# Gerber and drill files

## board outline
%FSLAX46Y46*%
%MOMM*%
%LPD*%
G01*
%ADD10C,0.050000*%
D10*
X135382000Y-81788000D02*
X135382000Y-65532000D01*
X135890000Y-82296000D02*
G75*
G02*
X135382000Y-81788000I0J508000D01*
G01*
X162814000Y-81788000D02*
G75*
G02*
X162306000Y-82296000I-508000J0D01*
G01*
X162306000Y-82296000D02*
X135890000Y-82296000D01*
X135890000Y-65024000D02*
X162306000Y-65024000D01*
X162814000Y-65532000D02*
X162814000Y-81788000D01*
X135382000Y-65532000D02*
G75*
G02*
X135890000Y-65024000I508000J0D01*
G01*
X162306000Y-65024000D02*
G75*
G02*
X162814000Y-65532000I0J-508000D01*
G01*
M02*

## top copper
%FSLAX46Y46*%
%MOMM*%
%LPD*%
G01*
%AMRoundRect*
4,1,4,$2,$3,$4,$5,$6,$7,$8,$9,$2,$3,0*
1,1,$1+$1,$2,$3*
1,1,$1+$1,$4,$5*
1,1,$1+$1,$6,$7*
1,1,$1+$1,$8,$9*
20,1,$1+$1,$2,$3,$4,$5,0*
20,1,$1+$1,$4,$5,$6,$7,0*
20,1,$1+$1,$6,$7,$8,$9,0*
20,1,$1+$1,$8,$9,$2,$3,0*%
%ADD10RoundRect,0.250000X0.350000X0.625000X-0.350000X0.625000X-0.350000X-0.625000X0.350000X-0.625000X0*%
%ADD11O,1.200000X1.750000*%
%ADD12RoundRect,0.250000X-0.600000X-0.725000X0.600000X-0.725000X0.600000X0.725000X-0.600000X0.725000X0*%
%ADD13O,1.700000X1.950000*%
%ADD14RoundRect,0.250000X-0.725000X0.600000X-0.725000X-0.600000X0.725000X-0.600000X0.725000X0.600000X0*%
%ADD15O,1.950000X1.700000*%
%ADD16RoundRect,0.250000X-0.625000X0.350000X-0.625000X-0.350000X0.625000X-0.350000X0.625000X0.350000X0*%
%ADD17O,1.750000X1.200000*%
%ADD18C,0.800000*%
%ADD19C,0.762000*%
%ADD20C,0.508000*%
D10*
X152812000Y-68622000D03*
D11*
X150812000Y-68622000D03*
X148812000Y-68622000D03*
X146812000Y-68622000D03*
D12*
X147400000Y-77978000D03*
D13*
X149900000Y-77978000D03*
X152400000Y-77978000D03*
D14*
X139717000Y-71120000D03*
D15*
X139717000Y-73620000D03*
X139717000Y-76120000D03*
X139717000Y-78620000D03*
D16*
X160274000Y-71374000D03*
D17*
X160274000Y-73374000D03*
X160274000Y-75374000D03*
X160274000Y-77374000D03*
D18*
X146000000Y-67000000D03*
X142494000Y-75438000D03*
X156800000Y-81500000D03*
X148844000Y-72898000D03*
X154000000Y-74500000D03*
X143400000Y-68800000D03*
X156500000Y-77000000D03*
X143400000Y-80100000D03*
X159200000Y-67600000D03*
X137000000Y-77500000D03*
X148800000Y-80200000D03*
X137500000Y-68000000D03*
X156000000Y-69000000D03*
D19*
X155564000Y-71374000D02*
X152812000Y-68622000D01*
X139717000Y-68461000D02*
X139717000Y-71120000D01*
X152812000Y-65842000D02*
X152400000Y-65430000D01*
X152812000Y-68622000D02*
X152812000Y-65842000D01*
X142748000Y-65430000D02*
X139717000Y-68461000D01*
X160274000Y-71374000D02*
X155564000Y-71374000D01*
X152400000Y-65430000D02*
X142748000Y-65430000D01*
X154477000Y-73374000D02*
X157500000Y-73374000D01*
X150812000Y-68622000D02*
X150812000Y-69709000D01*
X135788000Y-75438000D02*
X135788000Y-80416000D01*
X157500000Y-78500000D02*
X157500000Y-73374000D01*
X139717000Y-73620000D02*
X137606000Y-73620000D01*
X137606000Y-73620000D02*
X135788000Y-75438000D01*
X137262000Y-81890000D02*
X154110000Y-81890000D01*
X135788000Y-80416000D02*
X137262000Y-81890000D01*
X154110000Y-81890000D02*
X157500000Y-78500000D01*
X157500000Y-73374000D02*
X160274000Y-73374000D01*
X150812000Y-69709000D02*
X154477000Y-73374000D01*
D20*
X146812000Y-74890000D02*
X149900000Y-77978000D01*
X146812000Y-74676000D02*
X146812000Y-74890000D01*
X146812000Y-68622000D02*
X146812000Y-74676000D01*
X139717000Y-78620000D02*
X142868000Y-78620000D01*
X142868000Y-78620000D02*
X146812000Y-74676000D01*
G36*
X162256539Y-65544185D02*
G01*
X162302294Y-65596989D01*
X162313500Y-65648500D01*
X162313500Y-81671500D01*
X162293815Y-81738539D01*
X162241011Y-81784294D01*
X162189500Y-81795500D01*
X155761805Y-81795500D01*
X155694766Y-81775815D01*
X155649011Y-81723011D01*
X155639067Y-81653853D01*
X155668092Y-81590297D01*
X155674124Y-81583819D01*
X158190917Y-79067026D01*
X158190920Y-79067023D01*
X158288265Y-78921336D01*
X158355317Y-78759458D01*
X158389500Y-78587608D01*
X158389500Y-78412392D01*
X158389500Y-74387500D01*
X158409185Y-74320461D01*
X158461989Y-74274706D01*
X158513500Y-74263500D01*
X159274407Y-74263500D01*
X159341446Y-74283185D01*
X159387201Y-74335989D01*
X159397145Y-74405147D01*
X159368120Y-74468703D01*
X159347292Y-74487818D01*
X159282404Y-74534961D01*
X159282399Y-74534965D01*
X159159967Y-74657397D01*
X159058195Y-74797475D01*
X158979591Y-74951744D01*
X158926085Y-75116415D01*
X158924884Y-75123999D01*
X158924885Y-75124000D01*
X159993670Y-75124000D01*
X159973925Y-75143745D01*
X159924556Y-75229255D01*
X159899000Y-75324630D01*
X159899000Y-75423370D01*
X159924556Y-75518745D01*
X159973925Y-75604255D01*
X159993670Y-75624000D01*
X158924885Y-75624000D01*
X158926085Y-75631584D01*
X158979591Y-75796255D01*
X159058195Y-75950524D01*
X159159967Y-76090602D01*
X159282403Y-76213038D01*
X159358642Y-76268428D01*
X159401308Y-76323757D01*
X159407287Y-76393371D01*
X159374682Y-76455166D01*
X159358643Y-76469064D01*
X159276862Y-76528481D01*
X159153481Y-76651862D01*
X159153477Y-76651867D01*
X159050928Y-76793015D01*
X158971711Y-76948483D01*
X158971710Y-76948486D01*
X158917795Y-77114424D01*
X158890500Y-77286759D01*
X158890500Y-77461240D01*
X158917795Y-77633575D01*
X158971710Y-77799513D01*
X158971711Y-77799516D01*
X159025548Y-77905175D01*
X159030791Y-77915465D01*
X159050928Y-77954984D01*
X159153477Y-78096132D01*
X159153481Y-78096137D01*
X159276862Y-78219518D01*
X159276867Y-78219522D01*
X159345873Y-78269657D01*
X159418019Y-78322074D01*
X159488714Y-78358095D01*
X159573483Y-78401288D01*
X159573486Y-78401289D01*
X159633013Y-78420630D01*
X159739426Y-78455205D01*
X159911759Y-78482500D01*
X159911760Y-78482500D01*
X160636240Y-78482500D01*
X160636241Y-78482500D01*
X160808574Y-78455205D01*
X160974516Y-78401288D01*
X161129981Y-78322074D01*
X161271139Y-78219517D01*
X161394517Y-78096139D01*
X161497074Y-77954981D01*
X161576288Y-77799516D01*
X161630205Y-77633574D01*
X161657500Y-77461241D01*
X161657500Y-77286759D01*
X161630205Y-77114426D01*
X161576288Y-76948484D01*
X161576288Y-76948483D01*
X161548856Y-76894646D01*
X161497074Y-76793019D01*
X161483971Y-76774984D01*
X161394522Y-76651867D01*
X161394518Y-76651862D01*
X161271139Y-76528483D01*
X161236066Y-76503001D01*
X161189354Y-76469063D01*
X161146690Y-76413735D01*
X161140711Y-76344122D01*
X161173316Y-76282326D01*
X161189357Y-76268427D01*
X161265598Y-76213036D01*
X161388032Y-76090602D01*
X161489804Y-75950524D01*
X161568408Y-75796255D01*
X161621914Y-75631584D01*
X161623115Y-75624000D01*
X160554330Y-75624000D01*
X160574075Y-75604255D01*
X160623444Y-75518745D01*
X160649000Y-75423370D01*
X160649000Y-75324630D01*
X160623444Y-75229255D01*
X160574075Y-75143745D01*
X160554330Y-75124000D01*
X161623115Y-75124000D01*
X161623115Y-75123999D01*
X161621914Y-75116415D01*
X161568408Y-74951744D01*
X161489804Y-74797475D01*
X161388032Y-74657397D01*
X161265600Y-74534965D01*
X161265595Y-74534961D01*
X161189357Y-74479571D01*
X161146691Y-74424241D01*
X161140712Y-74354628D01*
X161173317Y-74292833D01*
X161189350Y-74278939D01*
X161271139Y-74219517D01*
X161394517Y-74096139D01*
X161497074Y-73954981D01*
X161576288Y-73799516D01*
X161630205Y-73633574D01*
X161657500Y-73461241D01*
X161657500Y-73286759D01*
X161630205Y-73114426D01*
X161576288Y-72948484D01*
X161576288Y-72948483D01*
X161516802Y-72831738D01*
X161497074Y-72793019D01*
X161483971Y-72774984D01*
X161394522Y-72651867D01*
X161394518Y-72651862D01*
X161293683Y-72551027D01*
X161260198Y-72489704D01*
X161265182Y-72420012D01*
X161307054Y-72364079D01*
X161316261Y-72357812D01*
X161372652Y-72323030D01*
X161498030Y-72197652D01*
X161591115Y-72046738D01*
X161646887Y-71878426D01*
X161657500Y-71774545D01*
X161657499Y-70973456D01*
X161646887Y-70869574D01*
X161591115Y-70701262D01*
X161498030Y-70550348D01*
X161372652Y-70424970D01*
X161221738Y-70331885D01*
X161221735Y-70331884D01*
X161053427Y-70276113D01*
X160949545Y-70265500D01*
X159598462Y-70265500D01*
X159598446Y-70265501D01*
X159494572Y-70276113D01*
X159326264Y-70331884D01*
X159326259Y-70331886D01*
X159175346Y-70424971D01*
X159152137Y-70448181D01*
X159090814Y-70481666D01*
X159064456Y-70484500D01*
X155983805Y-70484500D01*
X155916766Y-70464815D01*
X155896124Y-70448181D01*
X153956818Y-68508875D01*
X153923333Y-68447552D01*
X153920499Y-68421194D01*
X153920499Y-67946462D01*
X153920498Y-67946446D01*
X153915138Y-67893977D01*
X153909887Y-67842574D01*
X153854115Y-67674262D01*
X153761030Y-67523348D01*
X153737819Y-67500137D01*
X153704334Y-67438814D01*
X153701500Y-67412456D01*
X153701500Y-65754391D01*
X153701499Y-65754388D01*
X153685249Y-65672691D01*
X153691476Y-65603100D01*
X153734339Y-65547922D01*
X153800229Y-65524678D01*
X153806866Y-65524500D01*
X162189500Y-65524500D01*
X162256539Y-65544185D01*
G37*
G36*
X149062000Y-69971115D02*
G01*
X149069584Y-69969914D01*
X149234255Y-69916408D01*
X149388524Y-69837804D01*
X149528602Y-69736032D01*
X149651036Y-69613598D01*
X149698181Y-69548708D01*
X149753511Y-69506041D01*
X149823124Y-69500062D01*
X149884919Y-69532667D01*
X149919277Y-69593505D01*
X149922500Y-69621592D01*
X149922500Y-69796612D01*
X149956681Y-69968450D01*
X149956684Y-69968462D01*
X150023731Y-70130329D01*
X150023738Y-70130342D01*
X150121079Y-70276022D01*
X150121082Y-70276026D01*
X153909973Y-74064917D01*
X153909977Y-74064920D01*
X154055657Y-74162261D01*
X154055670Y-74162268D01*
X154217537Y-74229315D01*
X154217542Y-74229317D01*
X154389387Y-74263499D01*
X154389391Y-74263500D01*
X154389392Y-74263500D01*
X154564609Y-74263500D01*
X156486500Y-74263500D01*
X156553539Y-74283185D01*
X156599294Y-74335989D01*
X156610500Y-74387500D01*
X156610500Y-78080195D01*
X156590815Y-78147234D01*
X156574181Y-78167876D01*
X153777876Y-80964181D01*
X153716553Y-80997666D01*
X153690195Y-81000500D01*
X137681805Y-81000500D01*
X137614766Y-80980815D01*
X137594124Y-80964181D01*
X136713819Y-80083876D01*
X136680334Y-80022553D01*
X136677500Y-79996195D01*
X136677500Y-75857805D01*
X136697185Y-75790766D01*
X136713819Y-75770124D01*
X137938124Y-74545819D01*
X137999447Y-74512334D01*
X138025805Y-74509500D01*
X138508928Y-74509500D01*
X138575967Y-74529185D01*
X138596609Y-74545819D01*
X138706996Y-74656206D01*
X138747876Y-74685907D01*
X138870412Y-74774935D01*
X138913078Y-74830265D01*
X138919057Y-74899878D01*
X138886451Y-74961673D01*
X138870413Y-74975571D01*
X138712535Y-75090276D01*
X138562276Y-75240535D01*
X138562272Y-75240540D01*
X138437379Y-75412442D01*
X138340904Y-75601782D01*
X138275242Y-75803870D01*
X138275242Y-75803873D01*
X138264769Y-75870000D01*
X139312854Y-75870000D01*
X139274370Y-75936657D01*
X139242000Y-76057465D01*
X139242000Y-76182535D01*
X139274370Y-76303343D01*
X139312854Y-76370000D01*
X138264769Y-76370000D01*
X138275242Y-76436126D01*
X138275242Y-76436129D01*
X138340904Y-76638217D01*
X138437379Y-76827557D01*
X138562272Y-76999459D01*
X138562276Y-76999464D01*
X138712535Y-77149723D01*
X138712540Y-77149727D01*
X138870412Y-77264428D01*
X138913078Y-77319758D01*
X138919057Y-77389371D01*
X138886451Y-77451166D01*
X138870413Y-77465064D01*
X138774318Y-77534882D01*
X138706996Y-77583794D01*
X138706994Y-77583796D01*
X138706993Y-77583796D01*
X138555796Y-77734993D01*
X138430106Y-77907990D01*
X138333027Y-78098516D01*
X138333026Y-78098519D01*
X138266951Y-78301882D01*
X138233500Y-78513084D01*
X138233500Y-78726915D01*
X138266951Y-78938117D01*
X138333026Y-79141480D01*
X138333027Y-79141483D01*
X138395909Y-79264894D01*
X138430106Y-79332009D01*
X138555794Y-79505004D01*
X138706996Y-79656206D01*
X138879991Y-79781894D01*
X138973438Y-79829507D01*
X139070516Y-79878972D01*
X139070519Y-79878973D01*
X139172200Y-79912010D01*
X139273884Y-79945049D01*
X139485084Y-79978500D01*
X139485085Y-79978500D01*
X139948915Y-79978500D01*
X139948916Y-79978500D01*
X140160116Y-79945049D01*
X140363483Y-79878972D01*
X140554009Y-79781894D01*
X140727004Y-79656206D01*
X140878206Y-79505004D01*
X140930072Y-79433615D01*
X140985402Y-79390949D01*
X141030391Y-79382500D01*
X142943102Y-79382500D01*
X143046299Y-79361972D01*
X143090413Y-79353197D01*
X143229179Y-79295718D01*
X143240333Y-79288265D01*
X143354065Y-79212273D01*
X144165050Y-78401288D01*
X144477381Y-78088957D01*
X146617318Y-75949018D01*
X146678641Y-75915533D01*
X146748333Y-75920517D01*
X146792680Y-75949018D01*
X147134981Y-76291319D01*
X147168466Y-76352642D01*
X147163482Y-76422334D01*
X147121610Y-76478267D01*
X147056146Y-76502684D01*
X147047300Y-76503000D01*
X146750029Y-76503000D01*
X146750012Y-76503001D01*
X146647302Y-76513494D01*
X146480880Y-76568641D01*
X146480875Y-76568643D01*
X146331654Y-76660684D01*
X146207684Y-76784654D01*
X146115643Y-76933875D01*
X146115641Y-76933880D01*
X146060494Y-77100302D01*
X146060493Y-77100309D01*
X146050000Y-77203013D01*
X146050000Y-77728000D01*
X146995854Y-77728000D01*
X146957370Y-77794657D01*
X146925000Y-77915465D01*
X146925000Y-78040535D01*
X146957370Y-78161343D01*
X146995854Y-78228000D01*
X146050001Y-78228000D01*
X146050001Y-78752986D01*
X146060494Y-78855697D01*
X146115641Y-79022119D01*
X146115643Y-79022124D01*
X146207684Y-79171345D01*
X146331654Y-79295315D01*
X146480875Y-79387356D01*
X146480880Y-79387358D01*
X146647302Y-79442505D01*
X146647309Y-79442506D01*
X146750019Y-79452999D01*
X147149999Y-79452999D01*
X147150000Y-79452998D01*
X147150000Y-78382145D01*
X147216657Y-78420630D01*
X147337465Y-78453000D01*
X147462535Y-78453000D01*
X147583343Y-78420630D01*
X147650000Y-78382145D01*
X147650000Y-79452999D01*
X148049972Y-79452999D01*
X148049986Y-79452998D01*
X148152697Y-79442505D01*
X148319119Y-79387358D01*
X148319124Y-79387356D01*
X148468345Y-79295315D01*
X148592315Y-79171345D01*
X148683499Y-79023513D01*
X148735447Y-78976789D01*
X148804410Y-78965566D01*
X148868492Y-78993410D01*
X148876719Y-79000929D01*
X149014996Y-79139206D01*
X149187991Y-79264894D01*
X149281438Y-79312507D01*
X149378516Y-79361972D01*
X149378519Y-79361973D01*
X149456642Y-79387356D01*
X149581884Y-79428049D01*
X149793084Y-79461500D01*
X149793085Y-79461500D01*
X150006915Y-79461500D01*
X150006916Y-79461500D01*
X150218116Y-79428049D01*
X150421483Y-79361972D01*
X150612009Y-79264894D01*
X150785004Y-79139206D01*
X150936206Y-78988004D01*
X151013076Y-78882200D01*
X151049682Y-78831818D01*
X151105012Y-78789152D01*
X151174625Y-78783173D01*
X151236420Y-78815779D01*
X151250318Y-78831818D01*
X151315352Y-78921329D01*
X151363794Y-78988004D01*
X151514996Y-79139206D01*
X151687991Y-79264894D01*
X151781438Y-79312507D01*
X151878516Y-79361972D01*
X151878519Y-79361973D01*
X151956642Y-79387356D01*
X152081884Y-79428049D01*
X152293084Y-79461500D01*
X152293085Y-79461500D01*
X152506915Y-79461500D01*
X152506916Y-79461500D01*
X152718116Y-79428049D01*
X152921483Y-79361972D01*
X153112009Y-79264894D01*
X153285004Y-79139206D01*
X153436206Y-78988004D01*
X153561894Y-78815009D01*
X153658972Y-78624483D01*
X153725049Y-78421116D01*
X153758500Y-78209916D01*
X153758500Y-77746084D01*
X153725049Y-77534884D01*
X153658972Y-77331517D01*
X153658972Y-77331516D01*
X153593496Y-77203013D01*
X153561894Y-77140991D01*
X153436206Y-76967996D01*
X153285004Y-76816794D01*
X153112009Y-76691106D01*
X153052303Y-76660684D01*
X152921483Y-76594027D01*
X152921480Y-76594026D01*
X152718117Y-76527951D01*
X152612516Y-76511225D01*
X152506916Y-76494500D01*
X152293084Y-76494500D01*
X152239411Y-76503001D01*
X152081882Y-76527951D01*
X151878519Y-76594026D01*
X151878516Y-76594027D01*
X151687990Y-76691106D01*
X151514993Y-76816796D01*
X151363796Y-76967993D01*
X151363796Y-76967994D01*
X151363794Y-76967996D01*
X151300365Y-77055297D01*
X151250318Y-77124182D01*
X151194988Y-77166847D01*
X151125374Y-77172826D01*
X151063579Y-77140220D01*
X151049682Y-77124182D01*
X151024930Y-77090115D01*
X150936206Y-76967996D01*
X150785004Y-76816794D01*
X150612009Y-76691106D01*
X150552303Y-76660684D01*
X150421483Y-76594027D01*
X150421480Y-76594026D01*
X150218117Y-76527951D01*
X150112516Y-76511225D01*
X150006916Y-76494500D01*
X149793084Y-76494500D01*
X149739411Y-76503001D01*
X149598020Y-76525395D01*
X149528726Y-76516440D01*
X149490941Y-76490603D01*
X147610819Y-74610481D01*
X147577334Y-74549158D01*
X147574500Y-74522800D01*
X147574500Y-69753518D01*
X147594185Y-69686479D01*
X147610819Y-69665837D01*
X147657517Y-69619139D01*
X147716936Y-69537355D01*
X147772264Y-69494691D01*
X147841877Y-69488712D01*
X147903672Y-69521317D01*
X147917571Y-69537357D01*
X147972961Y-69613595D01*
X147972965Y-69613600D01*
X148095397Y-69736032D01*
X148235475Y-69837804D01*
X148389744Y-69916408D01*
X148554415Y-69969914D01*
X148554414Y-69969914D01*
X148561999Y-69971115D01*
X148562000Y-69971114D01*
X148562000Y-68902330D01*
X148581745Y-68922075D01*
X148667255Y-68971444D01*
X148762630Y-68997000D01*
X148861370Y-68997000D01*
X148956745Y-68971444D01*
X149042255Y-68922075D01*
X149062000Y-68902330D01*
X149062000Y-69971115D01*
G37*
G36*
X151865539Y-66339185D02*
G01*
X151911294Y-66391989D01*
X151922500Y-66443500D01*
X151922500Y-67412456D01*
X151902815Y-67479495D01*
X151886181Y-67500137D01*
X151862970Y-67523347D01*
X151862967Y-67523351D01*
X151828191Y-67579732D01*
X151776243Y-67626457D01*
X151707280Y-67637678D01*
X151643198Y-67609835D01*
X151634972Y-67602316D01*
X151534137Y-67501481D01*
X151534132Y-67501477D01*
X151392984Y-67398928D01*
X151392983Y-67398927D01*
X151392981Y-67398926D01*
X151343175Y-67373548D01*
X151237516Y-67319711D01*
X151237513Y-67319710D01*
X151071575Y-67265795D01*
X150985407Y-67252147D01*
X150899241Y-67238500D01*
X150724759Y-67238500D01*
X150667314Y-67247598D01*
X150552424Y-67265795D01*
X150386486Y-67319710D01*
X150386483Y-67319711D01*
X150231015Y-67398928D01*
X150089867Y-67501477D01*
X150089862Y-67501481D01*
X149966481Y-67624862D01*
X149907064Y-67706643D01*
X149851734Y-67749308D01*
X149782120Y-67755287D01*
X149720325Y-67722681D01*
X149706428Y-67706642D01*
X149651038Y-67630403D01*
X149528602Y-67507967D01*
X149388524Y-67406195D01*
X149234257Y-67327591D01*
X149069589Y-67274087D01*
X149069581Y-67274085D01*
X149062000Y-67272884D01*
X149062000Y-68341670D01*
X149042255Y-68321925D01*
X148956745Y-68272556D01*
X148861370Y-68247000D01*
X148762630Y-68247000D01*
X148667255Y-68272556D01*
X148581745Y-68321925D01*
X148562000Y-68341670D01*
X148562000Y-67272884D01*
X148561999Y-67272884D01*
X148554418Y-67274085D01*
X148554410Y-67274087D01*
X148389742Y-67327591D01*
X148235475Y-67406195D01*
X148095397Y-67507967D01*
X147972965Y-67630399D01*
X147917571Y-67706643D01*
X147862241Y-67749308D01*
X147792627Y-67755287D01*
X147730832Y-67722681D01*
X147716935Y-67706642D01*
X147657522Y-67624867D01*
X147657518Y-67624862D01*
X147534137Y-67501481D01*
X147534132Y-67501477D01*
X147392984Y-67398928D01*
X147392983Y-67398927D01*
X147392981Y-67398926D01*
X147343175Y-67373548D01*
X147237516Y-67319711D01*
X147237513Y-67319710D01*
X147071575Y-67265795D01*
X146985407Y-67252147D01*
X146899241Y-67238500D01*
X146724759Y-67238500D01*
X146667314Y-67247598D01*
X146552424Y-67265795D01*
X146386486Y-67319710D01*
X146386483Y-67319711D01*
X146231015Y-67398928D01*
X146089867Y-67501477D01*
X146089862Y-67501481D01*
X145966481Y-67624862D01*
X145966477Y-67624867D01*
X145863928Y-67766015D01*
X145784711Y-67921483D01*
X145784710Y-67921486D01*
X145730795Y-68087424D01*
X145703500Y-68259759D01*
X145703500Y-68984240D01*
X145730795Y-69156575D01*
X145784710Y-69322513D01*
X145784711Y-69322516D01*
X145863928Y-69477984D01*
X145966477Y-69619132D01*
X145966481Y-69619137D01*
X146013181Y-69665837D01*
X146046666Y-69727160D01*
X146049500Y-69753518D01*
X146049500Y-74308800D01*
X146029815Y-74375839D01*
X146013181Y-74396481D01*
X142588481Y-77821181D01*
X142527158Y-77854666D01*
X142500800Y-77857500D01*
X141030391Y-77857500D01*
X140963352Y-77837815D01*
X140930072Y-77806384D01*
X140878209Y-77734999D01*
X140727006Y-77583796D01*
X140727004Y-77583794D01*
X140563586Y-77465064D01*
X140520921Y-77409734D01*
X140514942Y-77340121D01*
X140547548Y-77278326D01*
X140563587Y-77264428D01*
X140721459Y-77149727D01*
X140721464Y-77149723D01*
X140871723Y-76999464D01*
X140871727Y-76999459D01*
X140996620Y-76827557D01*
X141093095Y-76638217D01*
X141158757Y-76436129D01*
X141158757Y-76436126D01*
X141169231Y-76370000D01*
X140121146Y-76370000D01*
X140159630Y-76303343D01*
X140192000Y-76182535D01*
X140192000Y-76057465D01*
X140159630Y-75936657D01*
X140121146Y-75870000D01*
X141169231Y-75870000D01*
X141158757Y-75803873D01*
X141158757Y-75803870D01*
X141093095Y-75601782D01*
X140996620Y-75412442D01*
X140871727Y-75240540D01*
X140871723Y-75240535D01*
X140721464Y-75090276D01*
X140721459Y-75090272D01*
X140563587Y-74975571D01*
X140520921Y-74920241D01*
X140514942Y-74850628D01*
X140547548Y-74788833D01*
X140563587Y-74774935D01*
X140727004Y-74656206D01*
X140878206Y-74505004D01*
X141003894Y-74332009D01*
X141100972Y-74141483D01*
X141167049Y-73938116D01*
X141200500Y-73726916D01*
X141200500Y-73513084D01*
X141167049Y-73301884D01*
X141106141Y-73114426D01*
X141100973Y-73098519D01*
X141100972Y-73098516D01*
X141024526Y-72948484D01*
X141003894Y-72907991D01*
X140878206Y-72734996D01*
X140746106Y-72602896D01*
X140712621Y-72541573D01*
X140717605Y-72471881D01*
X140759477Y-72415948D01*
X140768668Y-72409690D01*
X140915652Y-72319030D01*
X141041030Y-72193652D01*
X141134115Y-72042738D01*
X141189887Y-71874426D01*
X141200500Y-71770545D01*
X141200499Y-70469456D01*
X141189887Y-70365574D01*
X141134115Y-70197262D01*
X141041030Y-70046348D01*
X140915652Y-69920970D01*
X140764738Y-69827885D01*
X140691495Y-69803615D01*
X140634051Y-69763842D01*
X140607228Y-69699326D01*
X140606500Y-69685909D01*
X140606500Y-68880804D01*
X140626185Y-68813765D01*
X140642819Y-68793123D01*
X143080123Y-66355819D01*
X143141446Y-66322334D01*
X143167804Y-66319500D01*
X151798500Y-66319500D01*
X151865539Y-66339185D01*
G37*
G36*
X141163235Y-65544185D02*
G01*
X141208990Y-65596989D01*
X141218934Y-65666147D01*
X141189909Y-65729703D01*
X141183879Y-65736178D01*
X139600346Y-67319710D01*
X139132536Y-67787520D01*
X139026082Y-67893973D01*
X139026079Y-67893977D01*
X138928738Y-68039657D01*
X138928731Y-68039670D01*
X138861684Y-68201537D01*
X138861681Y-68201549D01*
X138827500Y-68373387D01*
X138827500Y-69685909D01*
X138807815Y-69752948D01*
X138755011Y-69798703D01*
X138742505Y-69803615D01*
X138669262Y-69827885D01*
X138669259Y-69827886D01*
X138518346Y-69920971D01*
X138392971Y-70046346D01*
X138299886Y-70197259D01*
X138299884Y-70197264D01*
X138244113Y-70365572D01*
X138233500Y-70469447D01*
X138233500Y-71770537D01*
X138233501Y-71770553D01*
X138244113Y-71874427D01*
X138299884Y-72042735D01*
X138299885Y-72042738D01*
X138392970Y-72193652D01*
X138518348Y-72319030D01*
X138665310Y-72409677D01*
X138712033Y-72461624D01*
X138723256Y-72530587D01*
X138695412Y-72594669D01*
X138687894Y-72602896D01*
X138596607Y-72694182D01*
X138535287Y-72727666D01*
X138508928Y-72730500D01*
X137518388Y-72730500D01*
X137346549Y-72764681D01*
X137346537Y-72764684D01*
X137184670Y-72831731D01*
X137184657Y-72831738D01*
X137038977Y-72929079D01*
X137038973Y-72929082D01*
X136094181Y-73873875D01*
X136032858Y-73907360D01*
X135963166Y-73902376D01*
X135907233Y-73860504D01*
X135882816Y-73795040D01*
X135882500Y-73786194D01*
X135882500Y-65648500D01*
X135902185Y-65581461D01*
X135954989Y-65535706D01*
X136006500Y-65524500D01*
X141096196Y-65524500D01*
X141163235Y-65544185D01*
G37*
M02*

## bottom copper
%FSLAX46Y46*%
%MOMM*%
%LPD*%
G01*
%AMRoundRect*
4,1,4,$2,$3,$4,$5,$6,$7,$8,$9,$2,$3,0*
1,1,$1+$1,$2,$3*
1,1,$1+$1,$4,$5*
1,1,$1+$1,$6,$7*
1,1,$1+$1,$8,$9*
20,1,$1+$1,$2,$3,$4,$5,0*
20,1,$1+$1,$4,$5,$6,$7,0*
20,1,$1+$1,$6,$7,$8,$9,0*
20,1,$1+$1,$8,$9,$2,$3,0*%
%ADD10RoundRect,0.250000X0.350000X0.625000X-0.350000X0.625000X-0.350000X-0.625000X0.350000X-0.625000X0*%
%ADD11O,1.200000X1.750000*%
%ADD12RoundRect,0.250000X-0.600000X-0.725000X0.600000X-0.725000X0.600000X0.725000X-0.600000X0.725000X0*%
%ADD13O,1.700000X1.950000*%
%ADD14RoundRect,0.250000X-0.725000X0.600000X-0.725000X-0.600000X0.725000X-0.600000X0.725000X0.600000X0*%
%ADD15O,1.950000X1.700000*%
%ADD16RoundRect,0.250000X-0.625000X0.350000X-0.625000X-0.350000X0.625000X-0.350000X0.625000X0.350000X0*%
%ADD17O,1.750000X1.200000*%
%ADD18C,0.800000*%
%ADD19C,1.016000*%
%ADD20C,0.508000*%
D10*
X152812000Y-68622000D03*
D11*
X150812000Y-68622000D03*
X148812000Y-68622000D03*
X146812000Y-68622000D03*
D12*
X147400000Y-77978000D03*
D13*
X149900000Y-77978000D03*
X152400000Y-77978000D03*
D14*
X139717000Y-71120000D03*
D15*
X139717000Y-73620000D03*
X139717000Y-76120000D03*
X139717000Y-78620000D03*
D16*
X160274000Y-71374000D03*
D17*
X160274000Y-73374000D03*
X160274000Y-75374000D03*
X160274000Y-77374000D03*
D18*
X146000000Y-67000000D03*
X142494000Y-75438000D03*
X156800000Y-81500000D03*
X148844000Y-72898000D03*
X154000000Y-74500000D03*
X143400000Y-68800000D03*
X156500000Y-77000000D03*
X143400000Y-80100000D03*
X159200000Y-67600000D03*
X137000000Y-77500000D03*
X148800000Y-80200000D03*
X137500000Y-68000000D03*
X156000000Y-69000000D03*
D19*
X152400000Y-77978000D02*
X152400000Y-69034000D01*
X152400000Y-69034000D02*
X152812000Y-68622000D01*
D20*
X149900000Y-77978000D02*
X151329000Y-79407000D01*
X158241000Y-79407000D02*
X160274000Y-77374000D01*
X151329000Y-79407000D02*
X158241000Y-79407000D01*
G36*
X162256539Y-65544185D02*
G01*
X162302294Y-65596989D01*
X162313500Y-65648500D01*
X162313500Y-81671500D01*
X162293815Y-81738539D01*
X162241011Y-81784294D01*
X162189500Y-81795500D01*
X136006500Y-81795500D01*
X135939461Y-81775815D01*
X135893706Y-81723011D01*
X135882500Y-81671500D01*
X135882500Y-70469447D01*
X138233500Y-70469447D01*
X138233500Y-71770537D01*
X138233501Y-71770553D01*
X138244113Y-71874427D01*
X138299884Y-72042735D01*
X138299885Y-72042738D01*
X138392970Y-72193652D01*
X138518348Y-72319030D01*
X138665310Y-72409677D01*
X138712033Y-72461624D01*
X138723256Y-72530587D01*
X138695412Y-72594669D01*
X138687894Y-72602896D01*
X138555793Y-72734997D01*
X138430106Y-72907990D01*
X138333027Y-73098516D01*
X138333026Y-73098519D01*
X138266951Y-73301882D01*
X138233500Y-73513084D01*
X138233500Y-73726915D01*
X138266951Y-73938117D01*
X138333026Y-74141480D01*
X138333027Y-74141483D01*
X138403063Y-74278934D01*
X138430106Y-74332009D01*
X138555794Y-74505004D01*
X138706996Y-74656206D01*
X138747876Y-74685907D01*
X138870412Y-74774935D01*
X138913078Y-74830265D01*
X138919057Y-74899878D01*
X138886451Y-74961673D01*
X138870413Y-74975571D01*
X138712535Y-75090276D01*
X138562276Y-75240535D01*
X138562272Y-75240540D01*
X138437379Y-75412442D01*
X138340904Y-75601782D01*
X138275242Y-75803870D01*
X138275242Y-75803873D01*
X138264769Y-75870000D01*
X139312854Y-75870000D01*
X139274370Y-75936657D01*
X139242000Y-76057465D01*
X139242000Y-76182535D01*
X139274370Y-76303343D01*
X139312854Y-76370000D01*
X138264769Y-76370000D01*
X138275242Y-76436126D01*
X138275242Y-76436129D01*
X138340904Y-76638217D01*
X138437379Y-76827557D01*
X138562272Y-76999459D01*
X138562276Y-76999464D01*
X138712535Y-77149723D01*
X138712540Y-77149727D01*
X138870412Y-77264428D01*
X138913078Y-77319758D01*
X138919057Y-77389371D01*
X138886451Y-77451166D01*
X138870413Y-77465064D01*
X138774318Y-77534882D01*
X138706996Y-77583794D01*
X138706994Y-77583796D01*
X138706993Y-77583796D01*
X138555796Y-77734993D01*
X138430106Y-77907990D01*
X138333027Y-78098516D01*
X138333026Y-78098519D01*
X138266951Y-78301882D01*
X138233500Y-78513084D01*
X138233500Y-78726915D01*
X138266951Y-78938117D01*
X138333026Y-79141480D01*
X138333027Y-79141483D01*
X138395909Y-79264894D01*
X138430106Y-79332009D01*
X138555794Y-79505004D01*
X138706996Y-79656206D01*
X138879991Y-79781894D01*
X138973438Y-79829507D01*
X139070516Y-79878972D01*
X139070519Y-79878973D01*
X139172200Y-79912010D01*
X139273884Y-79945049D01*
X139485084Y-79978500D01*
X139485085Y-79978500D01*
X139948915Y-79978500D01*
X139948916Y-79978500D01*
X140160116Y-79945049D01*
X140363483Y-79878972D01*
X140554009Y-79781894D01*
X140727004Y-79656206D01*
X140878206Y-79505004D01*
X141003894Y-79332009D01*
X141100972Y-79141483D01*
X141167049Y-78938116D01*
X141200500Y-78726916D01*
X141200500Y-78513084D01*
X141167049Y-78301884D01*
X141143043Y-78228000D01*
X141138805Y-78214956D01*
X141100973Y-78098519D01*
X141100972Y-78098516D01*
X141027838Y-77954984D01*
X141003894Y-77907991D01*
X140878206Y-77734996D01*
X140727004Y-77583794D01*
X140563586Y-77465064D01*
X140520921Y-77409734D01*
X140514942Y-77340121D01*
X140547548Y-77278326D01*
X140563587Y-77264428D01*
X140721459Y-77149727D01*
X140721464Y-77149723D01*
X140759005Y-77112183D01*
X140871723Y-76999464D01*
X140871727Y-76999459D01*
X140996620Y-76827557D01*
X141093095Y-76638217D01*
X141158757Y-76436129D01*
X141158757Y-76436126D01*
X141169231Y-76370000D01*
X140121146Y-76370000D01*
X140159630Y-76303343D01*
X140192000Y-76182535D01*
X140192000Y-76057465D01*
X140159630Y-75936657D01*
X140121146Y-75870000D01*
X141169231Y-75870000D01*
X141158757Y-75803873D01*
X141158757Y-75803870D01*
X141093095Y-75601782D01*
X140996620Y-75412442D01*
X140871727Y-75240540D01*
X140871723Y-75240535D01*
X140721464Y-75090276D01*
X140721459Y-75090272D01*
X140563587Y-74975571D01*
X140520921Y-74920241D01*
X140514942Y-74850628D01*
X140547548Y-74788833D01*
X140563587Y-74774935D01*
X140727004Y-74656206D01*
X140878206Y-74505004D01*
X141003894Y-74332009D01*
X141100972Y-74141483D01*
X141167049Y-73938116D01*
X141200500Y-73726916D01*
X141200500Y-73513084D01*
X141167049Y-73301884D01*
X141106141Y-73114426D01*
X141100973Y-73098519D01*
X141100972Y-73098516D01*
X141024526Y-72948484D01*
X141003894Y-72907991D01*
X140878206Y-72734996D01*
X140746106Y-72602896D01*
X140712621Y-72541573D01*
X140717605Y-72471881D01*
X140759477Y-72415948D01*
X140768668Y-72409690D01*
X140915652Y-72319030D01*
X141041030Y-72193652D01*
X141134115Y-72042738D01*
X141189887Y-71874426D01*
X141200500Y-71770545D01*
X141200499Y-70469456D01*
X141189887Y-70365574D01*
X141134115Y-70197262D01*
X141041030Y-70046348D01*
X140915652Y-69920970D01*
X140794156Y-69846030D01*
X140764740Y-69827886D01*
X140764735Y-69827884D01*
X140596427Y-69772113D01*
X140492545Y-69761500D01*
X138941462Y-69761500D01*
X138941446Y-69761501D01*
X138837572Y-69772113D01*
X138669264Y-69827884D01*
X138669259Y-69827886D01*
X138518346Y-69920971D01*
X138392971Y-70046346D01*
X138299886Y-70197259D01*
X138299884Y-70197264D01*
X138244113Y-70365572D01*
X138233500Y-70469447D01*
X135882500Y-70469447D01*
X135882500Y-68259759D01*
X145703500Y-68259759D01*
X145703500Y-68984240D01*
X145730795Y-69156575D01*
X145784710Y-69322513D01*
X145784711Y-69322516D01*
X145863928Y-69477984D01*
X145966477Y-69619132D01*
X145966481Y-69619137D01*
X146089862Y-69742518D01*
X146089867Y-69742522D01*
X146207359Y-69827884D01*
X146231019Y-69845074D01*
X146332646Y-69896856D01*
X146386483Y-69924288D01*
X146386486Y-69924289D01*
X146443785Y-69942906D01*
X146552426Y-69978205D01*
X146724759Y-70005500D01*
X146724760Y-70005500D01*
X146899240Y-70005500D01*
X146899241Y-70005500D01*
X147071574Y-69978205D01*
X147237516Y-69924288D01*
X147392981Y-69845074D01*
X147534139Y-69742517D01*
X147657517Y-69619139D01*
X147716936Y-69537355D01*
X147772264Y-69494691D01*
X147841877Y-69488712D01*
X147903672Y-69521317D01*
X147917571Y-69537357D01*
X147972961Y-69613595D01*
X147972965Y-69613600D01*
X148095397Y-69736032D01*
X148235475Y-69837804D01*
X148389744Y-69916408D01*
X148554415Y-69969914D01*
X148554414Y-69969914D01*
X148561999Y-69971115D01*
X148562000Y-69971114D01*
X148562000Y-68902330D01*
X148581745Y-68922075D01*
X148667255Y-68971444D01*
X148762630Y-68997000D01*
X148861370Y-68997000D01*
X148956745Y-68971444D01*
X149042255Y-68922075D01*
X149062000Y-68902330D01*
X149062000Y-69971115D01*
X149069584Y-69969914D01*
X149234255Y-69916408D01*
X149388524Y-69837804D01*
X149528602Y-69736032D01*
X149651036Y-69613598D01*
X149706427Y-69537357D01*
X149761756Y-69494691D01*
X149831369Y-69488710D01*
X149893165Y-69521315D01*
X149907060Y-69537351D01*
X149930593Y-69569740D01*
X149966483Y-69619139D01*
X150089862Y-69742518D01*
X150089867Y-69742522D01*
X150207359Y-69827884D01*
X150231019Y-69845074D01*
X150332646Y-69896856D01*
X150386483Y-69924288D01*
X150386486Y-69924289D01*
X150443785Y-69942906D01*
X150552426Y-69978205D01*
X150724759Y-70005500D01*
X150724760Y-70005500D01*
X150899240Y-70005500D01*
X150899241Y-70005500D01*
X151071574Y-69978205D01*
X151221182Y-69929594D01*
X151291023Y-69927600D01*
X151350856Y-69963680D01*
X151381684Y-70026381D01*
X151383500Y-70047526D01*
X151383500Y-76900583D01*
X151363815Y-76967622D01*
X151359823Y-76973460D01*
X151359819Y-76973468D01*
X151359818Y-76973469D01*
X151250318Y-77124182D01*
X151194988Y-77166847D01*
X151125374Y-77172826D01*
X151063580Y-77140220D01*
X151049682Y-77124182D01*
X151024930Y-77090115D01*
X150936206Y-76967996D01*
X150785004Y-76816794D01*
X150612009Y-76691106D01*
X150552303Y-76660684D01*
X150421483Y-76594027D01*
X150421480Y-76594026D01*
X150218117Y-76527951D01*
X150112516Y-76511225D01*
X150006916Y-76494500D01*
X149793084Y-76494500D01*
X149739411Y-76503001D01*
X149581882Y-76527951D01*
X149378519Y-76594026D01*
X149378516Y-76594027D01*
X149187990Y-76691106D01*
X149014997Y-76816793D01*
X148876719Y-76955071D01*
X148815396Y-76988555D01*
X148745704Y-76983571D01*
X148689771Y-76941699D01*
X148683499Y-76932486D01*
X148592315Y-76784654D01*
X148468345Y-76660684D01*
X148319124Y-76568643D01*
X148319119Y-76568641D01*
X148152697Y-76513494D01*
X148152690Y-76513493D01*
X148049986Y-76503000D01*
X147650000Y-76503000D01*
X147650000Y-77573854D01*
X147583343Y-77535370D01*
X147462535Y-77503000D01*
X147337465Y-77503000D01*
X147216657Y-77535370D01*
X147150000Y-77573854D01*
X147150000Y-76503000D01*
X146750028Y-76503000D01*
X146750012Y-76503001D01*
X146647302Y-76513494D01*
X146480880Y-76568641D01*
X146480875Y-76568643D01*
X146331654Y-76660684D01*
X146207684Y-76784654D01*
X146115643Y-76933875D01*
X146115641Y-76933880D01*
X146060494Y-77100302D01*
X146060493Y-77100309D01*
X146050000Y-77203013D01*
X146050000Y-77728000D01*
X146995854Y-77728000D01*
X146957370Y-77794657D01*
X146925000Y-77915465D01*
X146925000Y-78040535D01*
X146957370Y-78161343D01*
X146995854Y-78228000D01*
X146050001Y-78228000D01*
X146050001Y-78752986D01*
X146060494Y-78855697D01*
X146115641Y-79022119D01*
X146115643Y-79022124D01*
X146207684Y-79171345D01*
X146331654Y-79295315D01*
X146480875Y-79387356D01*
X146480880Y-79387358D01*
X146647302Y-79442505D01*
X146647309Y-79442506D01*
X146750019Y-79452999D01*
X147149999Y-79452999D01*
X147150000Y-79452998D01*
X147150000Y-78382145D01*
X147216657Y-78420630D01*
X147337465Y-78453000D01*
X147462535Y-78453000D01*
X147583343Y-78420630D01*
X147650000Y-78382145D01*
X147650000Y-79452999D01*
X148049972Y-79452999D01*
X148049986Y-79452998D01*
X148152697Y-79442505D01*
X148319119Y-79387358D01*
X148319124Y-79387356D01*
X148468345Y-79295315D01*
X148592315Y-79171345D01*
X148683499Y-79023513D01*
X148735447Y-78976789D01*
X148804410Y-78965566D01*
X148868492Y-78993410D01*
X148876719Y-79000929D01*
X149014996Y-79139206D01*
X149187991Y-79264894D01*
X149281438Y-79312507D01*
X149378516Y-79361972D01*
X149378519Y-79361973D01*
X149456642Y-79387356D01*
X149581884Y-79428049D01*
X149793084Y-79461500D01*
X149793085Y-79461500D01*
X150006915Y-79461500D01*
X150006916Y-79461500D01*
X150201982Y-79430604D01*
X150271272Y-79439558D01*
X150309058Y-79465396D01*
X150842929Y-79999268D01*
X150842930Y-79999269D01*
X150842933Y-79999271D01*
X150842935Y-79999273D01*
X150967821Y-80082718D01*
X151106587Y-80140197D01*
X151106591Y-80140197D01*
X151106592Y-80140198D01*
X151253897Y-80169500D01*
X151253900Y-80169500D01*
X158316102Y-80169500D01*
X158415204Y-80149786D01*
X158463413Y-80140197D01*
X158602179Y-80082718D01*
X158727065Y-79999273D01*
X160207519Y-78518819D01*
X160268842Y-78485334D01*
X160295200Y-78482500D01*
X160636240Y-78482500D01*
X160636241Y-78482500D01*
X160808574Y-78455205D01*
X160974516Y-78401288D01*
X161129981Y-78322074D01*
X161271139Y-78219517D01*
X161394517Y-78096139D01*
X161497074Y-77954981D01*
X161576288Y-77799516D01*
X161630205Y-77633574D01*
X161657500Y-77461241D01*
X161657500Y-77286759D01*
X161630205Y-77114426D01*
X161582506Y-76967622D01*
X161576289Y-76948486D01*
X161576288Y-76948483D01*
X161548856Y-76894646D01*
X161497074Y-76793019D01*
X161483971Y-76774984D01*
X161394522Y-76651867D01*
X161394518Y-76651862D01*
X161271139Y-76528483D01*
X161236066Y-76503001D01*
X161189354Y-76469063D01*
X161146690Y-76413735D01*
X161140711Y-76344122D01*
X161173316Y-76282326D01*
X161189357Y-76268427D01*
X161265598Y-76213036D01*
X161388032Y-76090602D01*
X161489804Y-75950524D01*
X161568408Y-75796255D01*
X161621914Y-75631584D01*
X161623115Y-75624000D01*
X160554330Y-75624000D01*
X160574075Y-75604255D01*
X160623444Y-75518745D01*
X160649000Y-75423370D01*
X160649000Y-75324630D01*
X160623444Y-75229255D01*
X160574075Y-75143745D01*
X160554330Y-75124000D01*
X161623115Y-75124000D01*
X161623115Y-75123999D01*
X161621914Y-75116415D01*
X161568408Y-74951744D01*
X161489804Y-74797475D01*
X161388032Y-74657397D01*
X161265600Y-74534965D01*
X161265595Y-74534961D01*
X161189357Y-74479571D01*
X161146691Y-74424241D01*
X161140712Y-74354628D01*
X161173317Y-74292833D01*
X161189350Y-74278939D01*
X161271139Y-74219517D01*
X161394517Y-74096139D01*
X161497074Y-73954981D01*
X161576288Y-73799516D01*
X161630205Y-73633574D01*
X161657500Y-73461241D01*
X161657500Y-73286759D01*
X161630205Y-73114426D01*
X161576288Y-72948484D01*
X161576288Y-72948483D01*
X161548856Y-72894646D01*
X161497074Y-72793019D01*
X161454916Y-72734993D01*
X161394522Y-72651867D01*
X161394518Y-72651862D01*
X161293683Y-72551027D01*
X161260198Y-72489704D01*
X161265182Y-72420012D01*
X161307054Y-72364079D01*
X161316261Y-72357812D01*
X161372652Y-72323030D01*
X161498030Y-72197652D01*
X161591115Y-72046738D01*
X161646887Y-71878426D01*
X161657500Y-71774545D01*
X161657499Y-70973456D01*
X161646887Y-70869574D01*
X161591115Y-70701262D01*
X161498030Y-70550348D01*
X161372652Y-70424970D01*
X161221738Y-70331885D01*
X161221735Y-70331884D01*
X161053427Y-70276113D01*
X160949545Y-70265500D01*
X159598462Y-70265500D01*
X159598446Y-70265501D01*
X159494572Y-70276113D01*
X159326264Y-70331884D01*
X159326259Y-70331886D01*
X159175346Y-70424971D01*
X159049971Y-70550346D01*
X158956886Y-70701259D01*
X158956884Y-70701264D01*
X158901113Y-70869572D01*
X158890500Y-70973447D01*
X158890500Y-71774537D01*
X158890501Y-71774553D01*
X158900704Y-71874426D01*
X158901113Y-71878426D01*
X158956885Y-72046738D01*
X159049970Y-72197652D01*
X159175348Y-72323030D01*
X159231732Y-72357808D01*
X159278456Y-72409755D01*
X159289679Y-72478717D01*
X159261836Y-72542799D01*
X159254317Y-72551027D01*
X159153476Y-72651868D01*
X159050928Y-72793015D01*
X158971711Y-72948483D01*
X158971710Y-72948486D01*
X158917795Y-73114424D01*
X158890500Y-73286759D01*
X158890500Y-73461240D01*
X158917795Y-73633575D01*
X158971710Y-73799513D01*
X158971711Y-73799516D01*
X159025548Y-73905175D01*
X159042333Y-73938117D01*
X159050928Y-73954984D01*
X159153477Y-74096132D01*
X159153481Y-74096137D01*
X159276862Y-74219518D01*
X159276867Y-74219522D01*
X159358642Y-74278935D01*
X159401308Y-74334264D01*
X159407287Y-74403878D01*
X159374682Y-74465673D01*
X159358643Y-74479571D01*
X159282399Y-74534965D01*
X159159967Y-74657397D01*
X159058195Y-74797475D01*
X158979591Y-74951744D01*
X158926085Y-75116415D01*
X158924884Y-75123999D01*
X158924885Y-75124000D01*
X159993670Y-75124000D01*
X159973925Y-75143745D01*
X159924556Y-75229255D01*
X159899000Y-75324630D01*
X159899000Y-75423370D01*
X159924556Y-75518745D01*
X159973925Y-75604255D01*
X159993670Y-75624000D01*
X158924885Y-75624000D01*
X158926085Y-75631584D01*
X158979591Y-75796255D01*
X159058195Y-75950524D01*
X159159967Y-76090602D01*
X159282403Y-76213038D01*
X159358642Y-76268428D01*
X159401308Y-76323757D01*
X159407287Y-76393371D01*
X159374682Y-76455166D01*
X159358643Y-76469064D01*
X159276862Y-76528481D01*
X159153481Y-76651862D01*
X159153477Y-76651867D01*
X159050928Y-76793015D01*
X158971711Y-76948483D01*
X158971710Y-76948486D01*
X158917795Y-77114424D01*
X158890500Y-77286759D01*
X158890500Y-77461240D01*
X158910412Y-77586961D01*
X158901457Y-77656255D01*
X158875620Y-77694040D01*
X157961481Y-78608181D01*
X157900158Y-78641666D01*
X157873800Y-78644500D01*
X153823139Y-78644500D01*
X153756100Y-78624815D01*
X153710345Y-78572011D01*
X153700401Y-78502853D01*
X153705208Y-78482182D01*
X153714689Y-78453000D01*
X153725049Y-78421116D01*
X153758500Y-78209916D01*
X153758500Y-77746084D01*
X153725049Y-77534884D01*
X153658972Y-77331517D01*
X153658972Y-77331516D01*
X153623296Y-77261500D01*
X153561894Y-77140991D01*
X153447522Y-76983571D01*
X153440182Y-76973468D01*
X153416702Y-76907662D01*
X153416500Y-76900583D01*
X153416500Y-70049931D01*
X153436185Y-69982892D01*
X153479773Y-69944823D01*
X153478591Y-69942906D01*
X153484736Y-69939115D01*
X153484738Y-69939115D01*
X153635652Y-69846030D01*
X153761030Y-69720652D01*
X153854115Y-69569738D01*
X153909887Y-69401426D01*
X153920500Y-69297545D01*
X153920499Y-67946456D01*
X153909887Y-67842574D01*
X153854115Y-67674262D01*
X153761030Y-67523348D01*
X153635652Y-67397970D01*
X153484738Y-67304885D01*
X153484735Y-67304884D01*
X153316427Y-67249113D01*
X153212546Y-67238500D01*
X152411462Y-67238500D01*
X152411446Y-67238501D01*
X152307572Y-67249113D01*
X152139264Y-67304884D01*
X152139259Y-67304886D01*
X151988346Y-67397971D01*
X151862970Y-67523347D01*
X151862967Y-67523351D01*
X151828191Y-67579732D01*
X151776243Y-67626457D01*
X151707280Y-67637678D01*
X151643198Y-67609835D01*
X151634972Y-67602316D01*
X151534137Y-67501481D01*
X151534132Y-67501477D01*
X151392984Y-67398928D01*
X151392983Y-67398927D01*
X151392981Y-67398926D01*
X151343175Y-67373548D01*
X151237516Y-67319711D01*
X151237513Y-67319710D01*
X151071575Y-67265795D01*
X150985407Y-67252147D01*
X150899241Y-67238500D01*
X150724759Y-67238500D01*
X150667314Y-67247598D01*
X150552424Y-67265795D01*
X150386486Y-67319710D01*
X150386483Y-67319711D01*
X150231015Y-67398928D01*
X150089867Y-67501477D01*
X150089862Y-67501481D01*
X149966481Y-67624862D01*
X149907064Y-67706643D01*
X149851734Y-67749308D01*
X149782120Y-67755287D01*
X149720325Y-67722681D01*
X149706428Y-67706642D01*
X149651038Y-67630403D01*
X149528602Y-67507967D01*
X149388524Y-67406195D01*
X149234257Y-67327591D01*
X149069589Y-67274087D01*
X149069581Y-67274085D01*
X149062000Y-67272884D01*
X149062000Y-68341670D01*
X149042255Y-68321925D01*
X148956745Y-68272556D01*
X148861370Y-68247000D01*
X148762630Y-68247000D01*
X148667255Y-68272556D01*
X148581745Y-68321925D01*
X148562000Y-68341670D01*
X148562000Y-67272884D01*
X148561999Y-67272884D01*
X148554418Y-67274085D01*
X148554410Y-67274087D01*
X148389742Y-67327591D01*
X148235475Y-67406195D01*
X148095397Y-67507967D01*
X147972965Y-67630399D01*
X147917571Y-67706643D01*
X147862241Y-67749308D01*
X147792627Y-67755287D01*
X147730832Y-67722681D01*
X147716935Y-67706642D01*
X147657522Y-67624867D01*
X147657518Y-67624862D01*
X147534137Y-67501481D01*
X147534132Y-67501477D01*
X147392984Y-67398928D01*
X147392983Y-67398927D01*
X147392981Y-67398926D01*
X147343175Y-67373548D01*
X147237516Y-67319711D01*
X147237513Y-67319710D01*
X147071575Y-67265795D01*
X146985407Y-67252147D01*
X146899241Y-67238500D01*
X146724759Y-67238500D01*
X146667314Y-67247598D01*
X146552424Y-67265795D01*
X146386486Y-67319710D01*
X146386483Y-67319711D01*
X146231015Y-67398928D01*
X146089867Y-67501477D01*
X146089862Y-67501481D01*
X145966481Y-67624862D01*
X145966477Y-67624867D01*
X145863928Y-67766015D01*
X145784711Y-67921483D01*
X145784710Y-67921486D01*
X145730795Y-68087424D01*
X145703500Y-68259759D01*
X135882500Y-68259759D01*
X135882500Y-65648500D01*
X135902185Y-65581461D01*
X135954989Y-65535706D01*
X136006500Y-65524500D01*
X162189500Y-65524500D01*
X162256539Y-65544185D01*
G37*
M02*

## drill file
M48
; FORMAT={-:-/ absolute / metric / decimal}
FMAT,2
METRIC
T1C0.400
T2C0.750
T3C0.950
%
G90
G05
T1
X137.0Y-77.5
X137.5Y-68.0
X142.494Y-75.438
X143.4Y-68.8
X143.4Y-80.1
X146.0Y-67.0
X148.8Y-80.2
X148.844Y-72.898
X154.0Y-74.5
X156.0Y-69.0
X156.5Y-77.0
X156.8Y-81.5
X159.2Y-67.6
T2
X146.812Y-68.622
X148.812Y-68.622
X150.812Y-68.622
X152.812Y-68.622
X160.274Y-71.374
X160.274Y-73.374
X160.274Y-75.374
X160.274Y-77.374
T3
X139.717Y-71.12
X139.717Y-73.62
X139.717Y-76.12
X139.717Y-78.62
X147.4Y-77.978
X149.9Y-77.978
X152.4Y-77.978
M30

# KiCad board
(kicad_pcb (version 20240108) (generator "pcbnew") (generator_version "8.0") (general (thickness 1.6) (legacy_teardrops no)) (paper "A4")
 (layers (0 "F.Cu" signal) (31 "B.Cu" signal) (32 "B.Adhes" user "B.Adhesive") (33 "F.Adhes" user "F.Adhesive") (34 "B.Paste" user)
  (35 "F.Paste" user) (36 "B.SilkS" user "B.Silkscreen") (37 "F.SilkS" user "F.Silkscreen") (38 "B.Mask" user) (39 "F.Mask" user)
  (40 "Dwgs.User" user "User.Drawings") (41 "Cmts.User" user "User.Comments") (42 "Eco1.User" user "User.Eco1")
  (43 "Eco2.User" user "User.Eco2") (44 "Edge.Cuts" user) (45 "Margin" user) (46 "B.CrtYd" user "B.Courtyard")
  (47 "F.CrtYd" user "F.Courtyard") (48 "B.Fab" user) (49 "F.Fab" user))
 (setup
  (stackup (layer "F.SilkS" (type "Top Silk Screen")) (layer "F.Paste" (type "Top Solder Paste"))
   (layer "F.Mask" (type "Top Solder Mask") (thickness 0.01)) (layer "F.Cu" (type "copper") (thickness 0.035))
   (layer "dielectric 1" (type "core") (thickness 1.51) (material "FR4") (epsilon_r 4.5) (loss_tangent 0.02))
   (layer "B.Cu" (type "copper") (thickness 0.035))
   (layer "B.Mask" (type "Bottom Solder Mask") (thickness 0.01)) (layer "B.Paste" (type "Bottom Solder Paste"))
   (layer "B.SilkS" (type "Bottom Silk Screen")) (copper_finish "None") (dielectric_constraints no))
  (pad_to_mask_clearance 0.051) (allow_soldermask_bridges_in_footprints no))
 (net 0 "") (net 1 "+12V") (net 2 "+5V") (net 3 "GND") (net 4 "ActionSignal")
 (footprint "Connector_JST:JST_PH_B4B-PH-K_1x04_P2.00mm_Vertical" (layer "F.Cu") (at 152.812 68.622 180)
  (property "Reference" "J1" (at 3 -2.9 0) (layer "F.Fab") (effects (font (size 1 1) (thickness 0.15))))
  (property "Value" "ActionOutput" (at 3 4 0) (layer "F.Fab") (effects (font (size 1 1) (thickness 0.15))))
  (pad "1" thru_hole roundrect (at 0 0 180) (size 1.2 1.75) (drill 0.75) (layers "*.Cu" "*.Mask") (remove_unused_layers no)
   (roundrect_rratio 0.208333) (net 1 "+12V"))
  (pad "2" thru_hole oval (at 2 0 180) (size 1.2 1.75) (drill 0.75) (layers "*.Cu" "*.Mask") (remove_unused_layers no) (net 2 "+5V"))
  (pad "3" thru_hole oval (at 4 0 180) (size 1.2 1.75) (drill 0.75) (layers "*.Cu" "*.Mask") (remove_unused_layers no) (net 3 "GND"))
  (pad "4" thru_hole oval (at 6 0 180) (size 1.2 1.75) (drill 0.75) (layers "*.Cu" "*.Mask") (remove_unused_layers no)
   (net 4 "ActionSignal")))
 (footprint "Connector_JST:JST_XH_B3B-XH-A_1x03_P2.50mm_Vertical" (layer "F.Cu") (at 147.4 77.978)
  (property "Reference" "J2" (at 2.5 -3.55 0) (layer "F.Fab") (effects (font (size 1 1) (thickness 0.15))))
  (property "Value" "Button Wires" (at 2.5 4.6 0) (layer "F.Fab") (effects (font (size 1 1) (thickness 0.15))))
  (pad "1" thru_hole roundrect (at 0 0) (size 1.7 1.95) (drill 0.95) (layers "*.Cu" "*.Mask") (remove_unused_layers no)
   (roundrect_rratio 0.147059) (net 3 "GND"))
  (pad "2" thru_hole oval (at 2.5 0) (size 1.7 1.95) (drill 0.95) (layers "*.Cu" "*.Mask") (remove_unused_layers no) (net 4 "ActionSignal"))
  (pad "3" thru_hole oval (at 5 0) (size 1.7 1.95) (drill 0.95) (layers "*.Cu" "*.Mask") (remove_unused_layers no) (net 1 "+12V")))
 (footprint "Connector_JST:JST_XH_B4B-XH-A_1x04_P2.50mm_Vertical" (layer "F.Cu") (at 139.717 71.12 -90)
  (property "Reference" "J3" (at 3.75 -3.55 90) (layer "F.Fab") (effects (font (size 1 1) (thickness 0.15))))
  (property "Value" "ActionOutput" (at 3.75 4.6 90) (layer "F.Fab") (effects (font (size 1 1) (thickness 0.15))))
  (pad "1" thru_hole roundrect (at 0 0 270) (size 1.7 1.95) (drill 0.95) (layers "*.Cu" "*.Mask") (remove_unused_layers no)
   (roundrect_rratio 0.147059) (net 1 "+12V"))
  (pad "2" thru_hole oval (at 2.5 0 270) (size 1.7 1.95) (drill 0.95) (layers "*.Cu" "*.Mask") (remove_unused_layers no) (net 2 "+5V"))
  (pad "3" thru_hole oval (at 5 0 270) (size 1.7 1.95) (drill 0.95) (layers "*.Cu" "*.Mask") (remove_unused_layers no) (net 3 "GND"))
  (pad "4" thru_hole oval (at 7.5 0 270) (size 1.7 1.95) (drill 0.95) (layers "*.Cu" "*.Mask") (remove_unused_layers no)
   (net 4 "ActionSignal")))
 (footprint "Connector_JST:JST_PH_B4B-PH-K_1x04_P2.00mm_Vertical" (layer "F.Cu") (at 160.274 71.374 -90)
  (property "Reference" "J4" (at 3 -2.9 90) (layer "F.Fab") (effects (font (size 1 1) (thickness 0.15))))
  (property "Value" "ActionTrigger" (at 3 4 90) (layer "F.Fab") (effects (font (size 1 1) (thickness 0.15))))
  (pad "1" thru_hole roundrect (at 0 0 270) (size 1.2 1.75) (drill 0.75) (layers "*.Cu" "*.Mask") (remove_unused_layers no)
   (roundrect_rratio 0.208333) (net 1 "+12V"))
  (pad "2" thru_hole oval (at 2 0 270) (size 1.2 1.75) (drill 0.75) (layers "*.Cu" "*.Mask") (remove_unused_layers no) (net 2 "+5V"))
  (pad "3" thru_hole oval (at 4 0 270) (size 1.2 1.75) (drill 0.75) (layers "*.Cu" "*.Mask") (remove_unused_layers no) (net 3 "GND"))
  (pad "4" thru_hole oval (at 6 0 270) (size 1.2 1.75) (drill 0.75) (layers "*.Cu" "*.Mask") (remove_unused_layers no)
   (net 4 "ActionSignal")))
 (gr_line (start 135.382 81.788) (end 135.382 65.532) (stroke (width 0.05) (type solid)) (layer "Edge.Cuts"))
 (gr_arc (start 135.89 82.296) (mid 135.53079 82.14721) (end 135.382 81.788) (stroke (width 0.05) (type default)) (layer "Edge.Cuts"))
 (gr_arc (start 162.814 81.788) (mid 162.66521 82.14721) (end 162.306 82.296) (stroke (width 0.05) (type default)) (layer "Edge.Cuts"))
 (gr_line (start 162.306 82.296) (end 135.89 82.296) (stroke (width 0.05) (type solid)) (layer "Edge.Cuts"))
 (gr_line (start 135.89 65.024) (end 162.306 65.024) (stroke (width 0.05) (type solid)) (layer "Edge.Cuts"))
 (gr_line (start 162.814 65.532) (end 162.814 81.788) (stroke (width 0.05) (type solid)) (layer "Edge.Cuts"))
 (gr_arc (start 135.382 65.532) (mid 135.53079 65.17279) (end 135.89 65.024) (stroke (width 0.05) (type default)) (layer "Edge.Cuts"))
 (gr_arc (start 162.306 65.024) (mid 162.66521 65.17279) (end 162.814 65.532) (stroke (width 0.05) (type default)) (layer "Edge.Cuts"))
 (segment (start 155.564 71.374) (end 152.812 68.622) (width 0.762) (layer "F.Cu") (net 1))
 (segment (start 139.717 68.461) (end 139.717 71.12) (width 0.762) (layer "F.Cu") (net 1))
 (segment (start 152.812 65.842) (end 152.4 65.43) (width 0.762) (layer "F.Cu") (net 1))
 (segment (start 152.812 68.622) (end 152.812 65.842) (width 0.762) (layer "F.Cu") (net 1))
 (segment (start 142.748 65.43) (end 139.717 68.461) (width 0.762) (layer "F.Cu") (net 1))
 (segment (start 160.274 71.374) (end 155.564 71.374) (width 0.762) (layer "F.Cu") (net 1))
 (segment (start 152.4 65.43) (end 142.748 65.43) (width 0.762) (layer "F.Cu") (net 1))
 (segment (start 152.4 77.978) (end 152.4 69.034) (width 1.016) (layer "B.Cu") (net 1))
 (segment (start 152.4 69.034) (end 152.812 68.622) (width 1.016) (layer "B.Cu") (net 1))
 (segment (start 154.477 73.374) (end 157.5 73.374) (width 0.762) (layer "F.Cu") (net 2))
 (segment (start 150.812 68.622) (end 150.812 69.709) (width 0.762) (layer "F.Cu") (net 2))
 (segment (start 135.788 75.438) (end 135.788 80.416) (width 0.762) (layer "F.Cu") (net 2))
 (segment (start 157.5 78.5) (end 157.5 73.374) (width 0.762) (layer "F.Cu") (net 2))
 (segment (start 139.717 73.62) (end 137.606 73.62) (width 0.762) (layer "F.Cu") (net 2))
 (segment (start 137.606 73.62) (end 135.788 75.438) (width 0.762) (layer "F.Cu") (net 2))
 (segment (start 137.262 81.89) (end 154.11 81.89) (width 0.762) (layer "F.Cu") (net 2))
 (segment (start 135.788 80.416) (end 137.262 81.89) (width 0.762) (layer "F.Cu") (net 2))
 (segment (start 154.11 81.89) (end 157.5 78.5) (width 0.762) (layer "F.Cu") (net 2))
 (segment (start 157.5 73.374) (end 160.274 73.374) (width 0.762) (layer "F.Cu") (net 2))
 (segment (start 150.812 69.709) (end 154.477 73.374) (width 0.762) (layer "F.Cu") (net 2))
 (via (at 146 67) (size 0.8) (drill 0.4) (layers "F.Cu" "B.Cu") (free yes) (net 3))
 (via (at 142.494 75.438) (size 0.8) (drill 0.4) (layers "F.Cu" "B.Cu") (free yes) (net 3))
 (via (at 156.8 81.5) (size 0.8) (drill 0.4) (layers "F.Cu" "B.Cu") (free yes) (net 3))
 (via (at 148.844 72.898) (size 0.8) (drill 0.4) (layers "F.Cu" "B.Cu") (free yes) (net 3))
 (via (at 154 74.5) (size 0.8) (drill 0.4) (layers "F.Cu" "B.Cu") (free yes) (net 3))
 (via (at 143.4 68.8) (size 0.8) (drill 0.4) (layers "F.Cu" "B.Cu") (free yes) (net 3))
 (via (at 156.5 77) (size 0.8) (drill 0.4) (layers "F.Cu" "B.Cu") (free yes) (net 3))
 (via (at 143.4 80.1) (size 0.8) (drill 0.4) (layers "F.Cu" "B.Cu") (free yes) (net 3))
 (via (at 159.2 67.6) (size 0.8) (drill 0.4) (layers "F.Cu" "B.Cu") (free yes) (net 3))
 (via (at 137 77.5) (size 0.8) (drill 0.4) (layers "F.Cu" "B.Cu") (free yes) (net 3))
 (via (at 148.8 80.2) (size 0.8) (drill 0.4) (layers "F.Cu" "B.Cu") (free yes) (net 3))
 (via (at 137.5 68) (size 0.8) (drill 0.4) (layers "F.Cu" "B.Cu") (free yes) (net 3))
 (via (at 156 69) (size 0.8) (drill 0.4) (layers "F.Cu" "B.Cu") (free yes) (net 3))
 (segment (start 146.812 74.89) (end 149.9 77.978) (width 0.508) (layer "F.Cu") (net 4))
 (segment (start 146.812 74.676) (end 146.812 74.89) (width 0.508) (layer "F.Cu") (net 4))
 (segment (start 146.812 68.622) (end 146.812 74.676) (width 0.508) (layer "F.Cu") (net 4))
 (segment (start 139.717 78.62) (end 142.868 78.62) (width 0.508) (layer "F.Cu") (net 4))
 (segment (start 142.868 78.62) (end 146.812 74.676) (width 0.508) (layer "F.Cu") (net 4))
 (segment (start 149.9 77.978) (end 151.329 79.407) (width 0.508) (layer "B.Cu") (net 4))
 (segment (start 158.241 79.407) (end 160.274 77.374) (width 0.508) (layer "B.Cu") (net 4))
 (segment (start 151.329 79.407) (end 158.241 79.407) (width 0.508) (layer "B.Cu") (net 4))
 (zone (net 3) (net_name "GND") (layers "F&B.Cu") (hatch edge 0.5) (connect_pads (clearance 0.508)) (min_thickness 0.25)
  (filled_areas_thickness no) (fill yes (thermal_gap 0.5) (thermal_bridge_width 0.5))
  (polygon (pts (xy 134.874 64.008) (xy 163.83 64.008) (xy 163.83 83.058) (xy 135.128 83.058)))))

